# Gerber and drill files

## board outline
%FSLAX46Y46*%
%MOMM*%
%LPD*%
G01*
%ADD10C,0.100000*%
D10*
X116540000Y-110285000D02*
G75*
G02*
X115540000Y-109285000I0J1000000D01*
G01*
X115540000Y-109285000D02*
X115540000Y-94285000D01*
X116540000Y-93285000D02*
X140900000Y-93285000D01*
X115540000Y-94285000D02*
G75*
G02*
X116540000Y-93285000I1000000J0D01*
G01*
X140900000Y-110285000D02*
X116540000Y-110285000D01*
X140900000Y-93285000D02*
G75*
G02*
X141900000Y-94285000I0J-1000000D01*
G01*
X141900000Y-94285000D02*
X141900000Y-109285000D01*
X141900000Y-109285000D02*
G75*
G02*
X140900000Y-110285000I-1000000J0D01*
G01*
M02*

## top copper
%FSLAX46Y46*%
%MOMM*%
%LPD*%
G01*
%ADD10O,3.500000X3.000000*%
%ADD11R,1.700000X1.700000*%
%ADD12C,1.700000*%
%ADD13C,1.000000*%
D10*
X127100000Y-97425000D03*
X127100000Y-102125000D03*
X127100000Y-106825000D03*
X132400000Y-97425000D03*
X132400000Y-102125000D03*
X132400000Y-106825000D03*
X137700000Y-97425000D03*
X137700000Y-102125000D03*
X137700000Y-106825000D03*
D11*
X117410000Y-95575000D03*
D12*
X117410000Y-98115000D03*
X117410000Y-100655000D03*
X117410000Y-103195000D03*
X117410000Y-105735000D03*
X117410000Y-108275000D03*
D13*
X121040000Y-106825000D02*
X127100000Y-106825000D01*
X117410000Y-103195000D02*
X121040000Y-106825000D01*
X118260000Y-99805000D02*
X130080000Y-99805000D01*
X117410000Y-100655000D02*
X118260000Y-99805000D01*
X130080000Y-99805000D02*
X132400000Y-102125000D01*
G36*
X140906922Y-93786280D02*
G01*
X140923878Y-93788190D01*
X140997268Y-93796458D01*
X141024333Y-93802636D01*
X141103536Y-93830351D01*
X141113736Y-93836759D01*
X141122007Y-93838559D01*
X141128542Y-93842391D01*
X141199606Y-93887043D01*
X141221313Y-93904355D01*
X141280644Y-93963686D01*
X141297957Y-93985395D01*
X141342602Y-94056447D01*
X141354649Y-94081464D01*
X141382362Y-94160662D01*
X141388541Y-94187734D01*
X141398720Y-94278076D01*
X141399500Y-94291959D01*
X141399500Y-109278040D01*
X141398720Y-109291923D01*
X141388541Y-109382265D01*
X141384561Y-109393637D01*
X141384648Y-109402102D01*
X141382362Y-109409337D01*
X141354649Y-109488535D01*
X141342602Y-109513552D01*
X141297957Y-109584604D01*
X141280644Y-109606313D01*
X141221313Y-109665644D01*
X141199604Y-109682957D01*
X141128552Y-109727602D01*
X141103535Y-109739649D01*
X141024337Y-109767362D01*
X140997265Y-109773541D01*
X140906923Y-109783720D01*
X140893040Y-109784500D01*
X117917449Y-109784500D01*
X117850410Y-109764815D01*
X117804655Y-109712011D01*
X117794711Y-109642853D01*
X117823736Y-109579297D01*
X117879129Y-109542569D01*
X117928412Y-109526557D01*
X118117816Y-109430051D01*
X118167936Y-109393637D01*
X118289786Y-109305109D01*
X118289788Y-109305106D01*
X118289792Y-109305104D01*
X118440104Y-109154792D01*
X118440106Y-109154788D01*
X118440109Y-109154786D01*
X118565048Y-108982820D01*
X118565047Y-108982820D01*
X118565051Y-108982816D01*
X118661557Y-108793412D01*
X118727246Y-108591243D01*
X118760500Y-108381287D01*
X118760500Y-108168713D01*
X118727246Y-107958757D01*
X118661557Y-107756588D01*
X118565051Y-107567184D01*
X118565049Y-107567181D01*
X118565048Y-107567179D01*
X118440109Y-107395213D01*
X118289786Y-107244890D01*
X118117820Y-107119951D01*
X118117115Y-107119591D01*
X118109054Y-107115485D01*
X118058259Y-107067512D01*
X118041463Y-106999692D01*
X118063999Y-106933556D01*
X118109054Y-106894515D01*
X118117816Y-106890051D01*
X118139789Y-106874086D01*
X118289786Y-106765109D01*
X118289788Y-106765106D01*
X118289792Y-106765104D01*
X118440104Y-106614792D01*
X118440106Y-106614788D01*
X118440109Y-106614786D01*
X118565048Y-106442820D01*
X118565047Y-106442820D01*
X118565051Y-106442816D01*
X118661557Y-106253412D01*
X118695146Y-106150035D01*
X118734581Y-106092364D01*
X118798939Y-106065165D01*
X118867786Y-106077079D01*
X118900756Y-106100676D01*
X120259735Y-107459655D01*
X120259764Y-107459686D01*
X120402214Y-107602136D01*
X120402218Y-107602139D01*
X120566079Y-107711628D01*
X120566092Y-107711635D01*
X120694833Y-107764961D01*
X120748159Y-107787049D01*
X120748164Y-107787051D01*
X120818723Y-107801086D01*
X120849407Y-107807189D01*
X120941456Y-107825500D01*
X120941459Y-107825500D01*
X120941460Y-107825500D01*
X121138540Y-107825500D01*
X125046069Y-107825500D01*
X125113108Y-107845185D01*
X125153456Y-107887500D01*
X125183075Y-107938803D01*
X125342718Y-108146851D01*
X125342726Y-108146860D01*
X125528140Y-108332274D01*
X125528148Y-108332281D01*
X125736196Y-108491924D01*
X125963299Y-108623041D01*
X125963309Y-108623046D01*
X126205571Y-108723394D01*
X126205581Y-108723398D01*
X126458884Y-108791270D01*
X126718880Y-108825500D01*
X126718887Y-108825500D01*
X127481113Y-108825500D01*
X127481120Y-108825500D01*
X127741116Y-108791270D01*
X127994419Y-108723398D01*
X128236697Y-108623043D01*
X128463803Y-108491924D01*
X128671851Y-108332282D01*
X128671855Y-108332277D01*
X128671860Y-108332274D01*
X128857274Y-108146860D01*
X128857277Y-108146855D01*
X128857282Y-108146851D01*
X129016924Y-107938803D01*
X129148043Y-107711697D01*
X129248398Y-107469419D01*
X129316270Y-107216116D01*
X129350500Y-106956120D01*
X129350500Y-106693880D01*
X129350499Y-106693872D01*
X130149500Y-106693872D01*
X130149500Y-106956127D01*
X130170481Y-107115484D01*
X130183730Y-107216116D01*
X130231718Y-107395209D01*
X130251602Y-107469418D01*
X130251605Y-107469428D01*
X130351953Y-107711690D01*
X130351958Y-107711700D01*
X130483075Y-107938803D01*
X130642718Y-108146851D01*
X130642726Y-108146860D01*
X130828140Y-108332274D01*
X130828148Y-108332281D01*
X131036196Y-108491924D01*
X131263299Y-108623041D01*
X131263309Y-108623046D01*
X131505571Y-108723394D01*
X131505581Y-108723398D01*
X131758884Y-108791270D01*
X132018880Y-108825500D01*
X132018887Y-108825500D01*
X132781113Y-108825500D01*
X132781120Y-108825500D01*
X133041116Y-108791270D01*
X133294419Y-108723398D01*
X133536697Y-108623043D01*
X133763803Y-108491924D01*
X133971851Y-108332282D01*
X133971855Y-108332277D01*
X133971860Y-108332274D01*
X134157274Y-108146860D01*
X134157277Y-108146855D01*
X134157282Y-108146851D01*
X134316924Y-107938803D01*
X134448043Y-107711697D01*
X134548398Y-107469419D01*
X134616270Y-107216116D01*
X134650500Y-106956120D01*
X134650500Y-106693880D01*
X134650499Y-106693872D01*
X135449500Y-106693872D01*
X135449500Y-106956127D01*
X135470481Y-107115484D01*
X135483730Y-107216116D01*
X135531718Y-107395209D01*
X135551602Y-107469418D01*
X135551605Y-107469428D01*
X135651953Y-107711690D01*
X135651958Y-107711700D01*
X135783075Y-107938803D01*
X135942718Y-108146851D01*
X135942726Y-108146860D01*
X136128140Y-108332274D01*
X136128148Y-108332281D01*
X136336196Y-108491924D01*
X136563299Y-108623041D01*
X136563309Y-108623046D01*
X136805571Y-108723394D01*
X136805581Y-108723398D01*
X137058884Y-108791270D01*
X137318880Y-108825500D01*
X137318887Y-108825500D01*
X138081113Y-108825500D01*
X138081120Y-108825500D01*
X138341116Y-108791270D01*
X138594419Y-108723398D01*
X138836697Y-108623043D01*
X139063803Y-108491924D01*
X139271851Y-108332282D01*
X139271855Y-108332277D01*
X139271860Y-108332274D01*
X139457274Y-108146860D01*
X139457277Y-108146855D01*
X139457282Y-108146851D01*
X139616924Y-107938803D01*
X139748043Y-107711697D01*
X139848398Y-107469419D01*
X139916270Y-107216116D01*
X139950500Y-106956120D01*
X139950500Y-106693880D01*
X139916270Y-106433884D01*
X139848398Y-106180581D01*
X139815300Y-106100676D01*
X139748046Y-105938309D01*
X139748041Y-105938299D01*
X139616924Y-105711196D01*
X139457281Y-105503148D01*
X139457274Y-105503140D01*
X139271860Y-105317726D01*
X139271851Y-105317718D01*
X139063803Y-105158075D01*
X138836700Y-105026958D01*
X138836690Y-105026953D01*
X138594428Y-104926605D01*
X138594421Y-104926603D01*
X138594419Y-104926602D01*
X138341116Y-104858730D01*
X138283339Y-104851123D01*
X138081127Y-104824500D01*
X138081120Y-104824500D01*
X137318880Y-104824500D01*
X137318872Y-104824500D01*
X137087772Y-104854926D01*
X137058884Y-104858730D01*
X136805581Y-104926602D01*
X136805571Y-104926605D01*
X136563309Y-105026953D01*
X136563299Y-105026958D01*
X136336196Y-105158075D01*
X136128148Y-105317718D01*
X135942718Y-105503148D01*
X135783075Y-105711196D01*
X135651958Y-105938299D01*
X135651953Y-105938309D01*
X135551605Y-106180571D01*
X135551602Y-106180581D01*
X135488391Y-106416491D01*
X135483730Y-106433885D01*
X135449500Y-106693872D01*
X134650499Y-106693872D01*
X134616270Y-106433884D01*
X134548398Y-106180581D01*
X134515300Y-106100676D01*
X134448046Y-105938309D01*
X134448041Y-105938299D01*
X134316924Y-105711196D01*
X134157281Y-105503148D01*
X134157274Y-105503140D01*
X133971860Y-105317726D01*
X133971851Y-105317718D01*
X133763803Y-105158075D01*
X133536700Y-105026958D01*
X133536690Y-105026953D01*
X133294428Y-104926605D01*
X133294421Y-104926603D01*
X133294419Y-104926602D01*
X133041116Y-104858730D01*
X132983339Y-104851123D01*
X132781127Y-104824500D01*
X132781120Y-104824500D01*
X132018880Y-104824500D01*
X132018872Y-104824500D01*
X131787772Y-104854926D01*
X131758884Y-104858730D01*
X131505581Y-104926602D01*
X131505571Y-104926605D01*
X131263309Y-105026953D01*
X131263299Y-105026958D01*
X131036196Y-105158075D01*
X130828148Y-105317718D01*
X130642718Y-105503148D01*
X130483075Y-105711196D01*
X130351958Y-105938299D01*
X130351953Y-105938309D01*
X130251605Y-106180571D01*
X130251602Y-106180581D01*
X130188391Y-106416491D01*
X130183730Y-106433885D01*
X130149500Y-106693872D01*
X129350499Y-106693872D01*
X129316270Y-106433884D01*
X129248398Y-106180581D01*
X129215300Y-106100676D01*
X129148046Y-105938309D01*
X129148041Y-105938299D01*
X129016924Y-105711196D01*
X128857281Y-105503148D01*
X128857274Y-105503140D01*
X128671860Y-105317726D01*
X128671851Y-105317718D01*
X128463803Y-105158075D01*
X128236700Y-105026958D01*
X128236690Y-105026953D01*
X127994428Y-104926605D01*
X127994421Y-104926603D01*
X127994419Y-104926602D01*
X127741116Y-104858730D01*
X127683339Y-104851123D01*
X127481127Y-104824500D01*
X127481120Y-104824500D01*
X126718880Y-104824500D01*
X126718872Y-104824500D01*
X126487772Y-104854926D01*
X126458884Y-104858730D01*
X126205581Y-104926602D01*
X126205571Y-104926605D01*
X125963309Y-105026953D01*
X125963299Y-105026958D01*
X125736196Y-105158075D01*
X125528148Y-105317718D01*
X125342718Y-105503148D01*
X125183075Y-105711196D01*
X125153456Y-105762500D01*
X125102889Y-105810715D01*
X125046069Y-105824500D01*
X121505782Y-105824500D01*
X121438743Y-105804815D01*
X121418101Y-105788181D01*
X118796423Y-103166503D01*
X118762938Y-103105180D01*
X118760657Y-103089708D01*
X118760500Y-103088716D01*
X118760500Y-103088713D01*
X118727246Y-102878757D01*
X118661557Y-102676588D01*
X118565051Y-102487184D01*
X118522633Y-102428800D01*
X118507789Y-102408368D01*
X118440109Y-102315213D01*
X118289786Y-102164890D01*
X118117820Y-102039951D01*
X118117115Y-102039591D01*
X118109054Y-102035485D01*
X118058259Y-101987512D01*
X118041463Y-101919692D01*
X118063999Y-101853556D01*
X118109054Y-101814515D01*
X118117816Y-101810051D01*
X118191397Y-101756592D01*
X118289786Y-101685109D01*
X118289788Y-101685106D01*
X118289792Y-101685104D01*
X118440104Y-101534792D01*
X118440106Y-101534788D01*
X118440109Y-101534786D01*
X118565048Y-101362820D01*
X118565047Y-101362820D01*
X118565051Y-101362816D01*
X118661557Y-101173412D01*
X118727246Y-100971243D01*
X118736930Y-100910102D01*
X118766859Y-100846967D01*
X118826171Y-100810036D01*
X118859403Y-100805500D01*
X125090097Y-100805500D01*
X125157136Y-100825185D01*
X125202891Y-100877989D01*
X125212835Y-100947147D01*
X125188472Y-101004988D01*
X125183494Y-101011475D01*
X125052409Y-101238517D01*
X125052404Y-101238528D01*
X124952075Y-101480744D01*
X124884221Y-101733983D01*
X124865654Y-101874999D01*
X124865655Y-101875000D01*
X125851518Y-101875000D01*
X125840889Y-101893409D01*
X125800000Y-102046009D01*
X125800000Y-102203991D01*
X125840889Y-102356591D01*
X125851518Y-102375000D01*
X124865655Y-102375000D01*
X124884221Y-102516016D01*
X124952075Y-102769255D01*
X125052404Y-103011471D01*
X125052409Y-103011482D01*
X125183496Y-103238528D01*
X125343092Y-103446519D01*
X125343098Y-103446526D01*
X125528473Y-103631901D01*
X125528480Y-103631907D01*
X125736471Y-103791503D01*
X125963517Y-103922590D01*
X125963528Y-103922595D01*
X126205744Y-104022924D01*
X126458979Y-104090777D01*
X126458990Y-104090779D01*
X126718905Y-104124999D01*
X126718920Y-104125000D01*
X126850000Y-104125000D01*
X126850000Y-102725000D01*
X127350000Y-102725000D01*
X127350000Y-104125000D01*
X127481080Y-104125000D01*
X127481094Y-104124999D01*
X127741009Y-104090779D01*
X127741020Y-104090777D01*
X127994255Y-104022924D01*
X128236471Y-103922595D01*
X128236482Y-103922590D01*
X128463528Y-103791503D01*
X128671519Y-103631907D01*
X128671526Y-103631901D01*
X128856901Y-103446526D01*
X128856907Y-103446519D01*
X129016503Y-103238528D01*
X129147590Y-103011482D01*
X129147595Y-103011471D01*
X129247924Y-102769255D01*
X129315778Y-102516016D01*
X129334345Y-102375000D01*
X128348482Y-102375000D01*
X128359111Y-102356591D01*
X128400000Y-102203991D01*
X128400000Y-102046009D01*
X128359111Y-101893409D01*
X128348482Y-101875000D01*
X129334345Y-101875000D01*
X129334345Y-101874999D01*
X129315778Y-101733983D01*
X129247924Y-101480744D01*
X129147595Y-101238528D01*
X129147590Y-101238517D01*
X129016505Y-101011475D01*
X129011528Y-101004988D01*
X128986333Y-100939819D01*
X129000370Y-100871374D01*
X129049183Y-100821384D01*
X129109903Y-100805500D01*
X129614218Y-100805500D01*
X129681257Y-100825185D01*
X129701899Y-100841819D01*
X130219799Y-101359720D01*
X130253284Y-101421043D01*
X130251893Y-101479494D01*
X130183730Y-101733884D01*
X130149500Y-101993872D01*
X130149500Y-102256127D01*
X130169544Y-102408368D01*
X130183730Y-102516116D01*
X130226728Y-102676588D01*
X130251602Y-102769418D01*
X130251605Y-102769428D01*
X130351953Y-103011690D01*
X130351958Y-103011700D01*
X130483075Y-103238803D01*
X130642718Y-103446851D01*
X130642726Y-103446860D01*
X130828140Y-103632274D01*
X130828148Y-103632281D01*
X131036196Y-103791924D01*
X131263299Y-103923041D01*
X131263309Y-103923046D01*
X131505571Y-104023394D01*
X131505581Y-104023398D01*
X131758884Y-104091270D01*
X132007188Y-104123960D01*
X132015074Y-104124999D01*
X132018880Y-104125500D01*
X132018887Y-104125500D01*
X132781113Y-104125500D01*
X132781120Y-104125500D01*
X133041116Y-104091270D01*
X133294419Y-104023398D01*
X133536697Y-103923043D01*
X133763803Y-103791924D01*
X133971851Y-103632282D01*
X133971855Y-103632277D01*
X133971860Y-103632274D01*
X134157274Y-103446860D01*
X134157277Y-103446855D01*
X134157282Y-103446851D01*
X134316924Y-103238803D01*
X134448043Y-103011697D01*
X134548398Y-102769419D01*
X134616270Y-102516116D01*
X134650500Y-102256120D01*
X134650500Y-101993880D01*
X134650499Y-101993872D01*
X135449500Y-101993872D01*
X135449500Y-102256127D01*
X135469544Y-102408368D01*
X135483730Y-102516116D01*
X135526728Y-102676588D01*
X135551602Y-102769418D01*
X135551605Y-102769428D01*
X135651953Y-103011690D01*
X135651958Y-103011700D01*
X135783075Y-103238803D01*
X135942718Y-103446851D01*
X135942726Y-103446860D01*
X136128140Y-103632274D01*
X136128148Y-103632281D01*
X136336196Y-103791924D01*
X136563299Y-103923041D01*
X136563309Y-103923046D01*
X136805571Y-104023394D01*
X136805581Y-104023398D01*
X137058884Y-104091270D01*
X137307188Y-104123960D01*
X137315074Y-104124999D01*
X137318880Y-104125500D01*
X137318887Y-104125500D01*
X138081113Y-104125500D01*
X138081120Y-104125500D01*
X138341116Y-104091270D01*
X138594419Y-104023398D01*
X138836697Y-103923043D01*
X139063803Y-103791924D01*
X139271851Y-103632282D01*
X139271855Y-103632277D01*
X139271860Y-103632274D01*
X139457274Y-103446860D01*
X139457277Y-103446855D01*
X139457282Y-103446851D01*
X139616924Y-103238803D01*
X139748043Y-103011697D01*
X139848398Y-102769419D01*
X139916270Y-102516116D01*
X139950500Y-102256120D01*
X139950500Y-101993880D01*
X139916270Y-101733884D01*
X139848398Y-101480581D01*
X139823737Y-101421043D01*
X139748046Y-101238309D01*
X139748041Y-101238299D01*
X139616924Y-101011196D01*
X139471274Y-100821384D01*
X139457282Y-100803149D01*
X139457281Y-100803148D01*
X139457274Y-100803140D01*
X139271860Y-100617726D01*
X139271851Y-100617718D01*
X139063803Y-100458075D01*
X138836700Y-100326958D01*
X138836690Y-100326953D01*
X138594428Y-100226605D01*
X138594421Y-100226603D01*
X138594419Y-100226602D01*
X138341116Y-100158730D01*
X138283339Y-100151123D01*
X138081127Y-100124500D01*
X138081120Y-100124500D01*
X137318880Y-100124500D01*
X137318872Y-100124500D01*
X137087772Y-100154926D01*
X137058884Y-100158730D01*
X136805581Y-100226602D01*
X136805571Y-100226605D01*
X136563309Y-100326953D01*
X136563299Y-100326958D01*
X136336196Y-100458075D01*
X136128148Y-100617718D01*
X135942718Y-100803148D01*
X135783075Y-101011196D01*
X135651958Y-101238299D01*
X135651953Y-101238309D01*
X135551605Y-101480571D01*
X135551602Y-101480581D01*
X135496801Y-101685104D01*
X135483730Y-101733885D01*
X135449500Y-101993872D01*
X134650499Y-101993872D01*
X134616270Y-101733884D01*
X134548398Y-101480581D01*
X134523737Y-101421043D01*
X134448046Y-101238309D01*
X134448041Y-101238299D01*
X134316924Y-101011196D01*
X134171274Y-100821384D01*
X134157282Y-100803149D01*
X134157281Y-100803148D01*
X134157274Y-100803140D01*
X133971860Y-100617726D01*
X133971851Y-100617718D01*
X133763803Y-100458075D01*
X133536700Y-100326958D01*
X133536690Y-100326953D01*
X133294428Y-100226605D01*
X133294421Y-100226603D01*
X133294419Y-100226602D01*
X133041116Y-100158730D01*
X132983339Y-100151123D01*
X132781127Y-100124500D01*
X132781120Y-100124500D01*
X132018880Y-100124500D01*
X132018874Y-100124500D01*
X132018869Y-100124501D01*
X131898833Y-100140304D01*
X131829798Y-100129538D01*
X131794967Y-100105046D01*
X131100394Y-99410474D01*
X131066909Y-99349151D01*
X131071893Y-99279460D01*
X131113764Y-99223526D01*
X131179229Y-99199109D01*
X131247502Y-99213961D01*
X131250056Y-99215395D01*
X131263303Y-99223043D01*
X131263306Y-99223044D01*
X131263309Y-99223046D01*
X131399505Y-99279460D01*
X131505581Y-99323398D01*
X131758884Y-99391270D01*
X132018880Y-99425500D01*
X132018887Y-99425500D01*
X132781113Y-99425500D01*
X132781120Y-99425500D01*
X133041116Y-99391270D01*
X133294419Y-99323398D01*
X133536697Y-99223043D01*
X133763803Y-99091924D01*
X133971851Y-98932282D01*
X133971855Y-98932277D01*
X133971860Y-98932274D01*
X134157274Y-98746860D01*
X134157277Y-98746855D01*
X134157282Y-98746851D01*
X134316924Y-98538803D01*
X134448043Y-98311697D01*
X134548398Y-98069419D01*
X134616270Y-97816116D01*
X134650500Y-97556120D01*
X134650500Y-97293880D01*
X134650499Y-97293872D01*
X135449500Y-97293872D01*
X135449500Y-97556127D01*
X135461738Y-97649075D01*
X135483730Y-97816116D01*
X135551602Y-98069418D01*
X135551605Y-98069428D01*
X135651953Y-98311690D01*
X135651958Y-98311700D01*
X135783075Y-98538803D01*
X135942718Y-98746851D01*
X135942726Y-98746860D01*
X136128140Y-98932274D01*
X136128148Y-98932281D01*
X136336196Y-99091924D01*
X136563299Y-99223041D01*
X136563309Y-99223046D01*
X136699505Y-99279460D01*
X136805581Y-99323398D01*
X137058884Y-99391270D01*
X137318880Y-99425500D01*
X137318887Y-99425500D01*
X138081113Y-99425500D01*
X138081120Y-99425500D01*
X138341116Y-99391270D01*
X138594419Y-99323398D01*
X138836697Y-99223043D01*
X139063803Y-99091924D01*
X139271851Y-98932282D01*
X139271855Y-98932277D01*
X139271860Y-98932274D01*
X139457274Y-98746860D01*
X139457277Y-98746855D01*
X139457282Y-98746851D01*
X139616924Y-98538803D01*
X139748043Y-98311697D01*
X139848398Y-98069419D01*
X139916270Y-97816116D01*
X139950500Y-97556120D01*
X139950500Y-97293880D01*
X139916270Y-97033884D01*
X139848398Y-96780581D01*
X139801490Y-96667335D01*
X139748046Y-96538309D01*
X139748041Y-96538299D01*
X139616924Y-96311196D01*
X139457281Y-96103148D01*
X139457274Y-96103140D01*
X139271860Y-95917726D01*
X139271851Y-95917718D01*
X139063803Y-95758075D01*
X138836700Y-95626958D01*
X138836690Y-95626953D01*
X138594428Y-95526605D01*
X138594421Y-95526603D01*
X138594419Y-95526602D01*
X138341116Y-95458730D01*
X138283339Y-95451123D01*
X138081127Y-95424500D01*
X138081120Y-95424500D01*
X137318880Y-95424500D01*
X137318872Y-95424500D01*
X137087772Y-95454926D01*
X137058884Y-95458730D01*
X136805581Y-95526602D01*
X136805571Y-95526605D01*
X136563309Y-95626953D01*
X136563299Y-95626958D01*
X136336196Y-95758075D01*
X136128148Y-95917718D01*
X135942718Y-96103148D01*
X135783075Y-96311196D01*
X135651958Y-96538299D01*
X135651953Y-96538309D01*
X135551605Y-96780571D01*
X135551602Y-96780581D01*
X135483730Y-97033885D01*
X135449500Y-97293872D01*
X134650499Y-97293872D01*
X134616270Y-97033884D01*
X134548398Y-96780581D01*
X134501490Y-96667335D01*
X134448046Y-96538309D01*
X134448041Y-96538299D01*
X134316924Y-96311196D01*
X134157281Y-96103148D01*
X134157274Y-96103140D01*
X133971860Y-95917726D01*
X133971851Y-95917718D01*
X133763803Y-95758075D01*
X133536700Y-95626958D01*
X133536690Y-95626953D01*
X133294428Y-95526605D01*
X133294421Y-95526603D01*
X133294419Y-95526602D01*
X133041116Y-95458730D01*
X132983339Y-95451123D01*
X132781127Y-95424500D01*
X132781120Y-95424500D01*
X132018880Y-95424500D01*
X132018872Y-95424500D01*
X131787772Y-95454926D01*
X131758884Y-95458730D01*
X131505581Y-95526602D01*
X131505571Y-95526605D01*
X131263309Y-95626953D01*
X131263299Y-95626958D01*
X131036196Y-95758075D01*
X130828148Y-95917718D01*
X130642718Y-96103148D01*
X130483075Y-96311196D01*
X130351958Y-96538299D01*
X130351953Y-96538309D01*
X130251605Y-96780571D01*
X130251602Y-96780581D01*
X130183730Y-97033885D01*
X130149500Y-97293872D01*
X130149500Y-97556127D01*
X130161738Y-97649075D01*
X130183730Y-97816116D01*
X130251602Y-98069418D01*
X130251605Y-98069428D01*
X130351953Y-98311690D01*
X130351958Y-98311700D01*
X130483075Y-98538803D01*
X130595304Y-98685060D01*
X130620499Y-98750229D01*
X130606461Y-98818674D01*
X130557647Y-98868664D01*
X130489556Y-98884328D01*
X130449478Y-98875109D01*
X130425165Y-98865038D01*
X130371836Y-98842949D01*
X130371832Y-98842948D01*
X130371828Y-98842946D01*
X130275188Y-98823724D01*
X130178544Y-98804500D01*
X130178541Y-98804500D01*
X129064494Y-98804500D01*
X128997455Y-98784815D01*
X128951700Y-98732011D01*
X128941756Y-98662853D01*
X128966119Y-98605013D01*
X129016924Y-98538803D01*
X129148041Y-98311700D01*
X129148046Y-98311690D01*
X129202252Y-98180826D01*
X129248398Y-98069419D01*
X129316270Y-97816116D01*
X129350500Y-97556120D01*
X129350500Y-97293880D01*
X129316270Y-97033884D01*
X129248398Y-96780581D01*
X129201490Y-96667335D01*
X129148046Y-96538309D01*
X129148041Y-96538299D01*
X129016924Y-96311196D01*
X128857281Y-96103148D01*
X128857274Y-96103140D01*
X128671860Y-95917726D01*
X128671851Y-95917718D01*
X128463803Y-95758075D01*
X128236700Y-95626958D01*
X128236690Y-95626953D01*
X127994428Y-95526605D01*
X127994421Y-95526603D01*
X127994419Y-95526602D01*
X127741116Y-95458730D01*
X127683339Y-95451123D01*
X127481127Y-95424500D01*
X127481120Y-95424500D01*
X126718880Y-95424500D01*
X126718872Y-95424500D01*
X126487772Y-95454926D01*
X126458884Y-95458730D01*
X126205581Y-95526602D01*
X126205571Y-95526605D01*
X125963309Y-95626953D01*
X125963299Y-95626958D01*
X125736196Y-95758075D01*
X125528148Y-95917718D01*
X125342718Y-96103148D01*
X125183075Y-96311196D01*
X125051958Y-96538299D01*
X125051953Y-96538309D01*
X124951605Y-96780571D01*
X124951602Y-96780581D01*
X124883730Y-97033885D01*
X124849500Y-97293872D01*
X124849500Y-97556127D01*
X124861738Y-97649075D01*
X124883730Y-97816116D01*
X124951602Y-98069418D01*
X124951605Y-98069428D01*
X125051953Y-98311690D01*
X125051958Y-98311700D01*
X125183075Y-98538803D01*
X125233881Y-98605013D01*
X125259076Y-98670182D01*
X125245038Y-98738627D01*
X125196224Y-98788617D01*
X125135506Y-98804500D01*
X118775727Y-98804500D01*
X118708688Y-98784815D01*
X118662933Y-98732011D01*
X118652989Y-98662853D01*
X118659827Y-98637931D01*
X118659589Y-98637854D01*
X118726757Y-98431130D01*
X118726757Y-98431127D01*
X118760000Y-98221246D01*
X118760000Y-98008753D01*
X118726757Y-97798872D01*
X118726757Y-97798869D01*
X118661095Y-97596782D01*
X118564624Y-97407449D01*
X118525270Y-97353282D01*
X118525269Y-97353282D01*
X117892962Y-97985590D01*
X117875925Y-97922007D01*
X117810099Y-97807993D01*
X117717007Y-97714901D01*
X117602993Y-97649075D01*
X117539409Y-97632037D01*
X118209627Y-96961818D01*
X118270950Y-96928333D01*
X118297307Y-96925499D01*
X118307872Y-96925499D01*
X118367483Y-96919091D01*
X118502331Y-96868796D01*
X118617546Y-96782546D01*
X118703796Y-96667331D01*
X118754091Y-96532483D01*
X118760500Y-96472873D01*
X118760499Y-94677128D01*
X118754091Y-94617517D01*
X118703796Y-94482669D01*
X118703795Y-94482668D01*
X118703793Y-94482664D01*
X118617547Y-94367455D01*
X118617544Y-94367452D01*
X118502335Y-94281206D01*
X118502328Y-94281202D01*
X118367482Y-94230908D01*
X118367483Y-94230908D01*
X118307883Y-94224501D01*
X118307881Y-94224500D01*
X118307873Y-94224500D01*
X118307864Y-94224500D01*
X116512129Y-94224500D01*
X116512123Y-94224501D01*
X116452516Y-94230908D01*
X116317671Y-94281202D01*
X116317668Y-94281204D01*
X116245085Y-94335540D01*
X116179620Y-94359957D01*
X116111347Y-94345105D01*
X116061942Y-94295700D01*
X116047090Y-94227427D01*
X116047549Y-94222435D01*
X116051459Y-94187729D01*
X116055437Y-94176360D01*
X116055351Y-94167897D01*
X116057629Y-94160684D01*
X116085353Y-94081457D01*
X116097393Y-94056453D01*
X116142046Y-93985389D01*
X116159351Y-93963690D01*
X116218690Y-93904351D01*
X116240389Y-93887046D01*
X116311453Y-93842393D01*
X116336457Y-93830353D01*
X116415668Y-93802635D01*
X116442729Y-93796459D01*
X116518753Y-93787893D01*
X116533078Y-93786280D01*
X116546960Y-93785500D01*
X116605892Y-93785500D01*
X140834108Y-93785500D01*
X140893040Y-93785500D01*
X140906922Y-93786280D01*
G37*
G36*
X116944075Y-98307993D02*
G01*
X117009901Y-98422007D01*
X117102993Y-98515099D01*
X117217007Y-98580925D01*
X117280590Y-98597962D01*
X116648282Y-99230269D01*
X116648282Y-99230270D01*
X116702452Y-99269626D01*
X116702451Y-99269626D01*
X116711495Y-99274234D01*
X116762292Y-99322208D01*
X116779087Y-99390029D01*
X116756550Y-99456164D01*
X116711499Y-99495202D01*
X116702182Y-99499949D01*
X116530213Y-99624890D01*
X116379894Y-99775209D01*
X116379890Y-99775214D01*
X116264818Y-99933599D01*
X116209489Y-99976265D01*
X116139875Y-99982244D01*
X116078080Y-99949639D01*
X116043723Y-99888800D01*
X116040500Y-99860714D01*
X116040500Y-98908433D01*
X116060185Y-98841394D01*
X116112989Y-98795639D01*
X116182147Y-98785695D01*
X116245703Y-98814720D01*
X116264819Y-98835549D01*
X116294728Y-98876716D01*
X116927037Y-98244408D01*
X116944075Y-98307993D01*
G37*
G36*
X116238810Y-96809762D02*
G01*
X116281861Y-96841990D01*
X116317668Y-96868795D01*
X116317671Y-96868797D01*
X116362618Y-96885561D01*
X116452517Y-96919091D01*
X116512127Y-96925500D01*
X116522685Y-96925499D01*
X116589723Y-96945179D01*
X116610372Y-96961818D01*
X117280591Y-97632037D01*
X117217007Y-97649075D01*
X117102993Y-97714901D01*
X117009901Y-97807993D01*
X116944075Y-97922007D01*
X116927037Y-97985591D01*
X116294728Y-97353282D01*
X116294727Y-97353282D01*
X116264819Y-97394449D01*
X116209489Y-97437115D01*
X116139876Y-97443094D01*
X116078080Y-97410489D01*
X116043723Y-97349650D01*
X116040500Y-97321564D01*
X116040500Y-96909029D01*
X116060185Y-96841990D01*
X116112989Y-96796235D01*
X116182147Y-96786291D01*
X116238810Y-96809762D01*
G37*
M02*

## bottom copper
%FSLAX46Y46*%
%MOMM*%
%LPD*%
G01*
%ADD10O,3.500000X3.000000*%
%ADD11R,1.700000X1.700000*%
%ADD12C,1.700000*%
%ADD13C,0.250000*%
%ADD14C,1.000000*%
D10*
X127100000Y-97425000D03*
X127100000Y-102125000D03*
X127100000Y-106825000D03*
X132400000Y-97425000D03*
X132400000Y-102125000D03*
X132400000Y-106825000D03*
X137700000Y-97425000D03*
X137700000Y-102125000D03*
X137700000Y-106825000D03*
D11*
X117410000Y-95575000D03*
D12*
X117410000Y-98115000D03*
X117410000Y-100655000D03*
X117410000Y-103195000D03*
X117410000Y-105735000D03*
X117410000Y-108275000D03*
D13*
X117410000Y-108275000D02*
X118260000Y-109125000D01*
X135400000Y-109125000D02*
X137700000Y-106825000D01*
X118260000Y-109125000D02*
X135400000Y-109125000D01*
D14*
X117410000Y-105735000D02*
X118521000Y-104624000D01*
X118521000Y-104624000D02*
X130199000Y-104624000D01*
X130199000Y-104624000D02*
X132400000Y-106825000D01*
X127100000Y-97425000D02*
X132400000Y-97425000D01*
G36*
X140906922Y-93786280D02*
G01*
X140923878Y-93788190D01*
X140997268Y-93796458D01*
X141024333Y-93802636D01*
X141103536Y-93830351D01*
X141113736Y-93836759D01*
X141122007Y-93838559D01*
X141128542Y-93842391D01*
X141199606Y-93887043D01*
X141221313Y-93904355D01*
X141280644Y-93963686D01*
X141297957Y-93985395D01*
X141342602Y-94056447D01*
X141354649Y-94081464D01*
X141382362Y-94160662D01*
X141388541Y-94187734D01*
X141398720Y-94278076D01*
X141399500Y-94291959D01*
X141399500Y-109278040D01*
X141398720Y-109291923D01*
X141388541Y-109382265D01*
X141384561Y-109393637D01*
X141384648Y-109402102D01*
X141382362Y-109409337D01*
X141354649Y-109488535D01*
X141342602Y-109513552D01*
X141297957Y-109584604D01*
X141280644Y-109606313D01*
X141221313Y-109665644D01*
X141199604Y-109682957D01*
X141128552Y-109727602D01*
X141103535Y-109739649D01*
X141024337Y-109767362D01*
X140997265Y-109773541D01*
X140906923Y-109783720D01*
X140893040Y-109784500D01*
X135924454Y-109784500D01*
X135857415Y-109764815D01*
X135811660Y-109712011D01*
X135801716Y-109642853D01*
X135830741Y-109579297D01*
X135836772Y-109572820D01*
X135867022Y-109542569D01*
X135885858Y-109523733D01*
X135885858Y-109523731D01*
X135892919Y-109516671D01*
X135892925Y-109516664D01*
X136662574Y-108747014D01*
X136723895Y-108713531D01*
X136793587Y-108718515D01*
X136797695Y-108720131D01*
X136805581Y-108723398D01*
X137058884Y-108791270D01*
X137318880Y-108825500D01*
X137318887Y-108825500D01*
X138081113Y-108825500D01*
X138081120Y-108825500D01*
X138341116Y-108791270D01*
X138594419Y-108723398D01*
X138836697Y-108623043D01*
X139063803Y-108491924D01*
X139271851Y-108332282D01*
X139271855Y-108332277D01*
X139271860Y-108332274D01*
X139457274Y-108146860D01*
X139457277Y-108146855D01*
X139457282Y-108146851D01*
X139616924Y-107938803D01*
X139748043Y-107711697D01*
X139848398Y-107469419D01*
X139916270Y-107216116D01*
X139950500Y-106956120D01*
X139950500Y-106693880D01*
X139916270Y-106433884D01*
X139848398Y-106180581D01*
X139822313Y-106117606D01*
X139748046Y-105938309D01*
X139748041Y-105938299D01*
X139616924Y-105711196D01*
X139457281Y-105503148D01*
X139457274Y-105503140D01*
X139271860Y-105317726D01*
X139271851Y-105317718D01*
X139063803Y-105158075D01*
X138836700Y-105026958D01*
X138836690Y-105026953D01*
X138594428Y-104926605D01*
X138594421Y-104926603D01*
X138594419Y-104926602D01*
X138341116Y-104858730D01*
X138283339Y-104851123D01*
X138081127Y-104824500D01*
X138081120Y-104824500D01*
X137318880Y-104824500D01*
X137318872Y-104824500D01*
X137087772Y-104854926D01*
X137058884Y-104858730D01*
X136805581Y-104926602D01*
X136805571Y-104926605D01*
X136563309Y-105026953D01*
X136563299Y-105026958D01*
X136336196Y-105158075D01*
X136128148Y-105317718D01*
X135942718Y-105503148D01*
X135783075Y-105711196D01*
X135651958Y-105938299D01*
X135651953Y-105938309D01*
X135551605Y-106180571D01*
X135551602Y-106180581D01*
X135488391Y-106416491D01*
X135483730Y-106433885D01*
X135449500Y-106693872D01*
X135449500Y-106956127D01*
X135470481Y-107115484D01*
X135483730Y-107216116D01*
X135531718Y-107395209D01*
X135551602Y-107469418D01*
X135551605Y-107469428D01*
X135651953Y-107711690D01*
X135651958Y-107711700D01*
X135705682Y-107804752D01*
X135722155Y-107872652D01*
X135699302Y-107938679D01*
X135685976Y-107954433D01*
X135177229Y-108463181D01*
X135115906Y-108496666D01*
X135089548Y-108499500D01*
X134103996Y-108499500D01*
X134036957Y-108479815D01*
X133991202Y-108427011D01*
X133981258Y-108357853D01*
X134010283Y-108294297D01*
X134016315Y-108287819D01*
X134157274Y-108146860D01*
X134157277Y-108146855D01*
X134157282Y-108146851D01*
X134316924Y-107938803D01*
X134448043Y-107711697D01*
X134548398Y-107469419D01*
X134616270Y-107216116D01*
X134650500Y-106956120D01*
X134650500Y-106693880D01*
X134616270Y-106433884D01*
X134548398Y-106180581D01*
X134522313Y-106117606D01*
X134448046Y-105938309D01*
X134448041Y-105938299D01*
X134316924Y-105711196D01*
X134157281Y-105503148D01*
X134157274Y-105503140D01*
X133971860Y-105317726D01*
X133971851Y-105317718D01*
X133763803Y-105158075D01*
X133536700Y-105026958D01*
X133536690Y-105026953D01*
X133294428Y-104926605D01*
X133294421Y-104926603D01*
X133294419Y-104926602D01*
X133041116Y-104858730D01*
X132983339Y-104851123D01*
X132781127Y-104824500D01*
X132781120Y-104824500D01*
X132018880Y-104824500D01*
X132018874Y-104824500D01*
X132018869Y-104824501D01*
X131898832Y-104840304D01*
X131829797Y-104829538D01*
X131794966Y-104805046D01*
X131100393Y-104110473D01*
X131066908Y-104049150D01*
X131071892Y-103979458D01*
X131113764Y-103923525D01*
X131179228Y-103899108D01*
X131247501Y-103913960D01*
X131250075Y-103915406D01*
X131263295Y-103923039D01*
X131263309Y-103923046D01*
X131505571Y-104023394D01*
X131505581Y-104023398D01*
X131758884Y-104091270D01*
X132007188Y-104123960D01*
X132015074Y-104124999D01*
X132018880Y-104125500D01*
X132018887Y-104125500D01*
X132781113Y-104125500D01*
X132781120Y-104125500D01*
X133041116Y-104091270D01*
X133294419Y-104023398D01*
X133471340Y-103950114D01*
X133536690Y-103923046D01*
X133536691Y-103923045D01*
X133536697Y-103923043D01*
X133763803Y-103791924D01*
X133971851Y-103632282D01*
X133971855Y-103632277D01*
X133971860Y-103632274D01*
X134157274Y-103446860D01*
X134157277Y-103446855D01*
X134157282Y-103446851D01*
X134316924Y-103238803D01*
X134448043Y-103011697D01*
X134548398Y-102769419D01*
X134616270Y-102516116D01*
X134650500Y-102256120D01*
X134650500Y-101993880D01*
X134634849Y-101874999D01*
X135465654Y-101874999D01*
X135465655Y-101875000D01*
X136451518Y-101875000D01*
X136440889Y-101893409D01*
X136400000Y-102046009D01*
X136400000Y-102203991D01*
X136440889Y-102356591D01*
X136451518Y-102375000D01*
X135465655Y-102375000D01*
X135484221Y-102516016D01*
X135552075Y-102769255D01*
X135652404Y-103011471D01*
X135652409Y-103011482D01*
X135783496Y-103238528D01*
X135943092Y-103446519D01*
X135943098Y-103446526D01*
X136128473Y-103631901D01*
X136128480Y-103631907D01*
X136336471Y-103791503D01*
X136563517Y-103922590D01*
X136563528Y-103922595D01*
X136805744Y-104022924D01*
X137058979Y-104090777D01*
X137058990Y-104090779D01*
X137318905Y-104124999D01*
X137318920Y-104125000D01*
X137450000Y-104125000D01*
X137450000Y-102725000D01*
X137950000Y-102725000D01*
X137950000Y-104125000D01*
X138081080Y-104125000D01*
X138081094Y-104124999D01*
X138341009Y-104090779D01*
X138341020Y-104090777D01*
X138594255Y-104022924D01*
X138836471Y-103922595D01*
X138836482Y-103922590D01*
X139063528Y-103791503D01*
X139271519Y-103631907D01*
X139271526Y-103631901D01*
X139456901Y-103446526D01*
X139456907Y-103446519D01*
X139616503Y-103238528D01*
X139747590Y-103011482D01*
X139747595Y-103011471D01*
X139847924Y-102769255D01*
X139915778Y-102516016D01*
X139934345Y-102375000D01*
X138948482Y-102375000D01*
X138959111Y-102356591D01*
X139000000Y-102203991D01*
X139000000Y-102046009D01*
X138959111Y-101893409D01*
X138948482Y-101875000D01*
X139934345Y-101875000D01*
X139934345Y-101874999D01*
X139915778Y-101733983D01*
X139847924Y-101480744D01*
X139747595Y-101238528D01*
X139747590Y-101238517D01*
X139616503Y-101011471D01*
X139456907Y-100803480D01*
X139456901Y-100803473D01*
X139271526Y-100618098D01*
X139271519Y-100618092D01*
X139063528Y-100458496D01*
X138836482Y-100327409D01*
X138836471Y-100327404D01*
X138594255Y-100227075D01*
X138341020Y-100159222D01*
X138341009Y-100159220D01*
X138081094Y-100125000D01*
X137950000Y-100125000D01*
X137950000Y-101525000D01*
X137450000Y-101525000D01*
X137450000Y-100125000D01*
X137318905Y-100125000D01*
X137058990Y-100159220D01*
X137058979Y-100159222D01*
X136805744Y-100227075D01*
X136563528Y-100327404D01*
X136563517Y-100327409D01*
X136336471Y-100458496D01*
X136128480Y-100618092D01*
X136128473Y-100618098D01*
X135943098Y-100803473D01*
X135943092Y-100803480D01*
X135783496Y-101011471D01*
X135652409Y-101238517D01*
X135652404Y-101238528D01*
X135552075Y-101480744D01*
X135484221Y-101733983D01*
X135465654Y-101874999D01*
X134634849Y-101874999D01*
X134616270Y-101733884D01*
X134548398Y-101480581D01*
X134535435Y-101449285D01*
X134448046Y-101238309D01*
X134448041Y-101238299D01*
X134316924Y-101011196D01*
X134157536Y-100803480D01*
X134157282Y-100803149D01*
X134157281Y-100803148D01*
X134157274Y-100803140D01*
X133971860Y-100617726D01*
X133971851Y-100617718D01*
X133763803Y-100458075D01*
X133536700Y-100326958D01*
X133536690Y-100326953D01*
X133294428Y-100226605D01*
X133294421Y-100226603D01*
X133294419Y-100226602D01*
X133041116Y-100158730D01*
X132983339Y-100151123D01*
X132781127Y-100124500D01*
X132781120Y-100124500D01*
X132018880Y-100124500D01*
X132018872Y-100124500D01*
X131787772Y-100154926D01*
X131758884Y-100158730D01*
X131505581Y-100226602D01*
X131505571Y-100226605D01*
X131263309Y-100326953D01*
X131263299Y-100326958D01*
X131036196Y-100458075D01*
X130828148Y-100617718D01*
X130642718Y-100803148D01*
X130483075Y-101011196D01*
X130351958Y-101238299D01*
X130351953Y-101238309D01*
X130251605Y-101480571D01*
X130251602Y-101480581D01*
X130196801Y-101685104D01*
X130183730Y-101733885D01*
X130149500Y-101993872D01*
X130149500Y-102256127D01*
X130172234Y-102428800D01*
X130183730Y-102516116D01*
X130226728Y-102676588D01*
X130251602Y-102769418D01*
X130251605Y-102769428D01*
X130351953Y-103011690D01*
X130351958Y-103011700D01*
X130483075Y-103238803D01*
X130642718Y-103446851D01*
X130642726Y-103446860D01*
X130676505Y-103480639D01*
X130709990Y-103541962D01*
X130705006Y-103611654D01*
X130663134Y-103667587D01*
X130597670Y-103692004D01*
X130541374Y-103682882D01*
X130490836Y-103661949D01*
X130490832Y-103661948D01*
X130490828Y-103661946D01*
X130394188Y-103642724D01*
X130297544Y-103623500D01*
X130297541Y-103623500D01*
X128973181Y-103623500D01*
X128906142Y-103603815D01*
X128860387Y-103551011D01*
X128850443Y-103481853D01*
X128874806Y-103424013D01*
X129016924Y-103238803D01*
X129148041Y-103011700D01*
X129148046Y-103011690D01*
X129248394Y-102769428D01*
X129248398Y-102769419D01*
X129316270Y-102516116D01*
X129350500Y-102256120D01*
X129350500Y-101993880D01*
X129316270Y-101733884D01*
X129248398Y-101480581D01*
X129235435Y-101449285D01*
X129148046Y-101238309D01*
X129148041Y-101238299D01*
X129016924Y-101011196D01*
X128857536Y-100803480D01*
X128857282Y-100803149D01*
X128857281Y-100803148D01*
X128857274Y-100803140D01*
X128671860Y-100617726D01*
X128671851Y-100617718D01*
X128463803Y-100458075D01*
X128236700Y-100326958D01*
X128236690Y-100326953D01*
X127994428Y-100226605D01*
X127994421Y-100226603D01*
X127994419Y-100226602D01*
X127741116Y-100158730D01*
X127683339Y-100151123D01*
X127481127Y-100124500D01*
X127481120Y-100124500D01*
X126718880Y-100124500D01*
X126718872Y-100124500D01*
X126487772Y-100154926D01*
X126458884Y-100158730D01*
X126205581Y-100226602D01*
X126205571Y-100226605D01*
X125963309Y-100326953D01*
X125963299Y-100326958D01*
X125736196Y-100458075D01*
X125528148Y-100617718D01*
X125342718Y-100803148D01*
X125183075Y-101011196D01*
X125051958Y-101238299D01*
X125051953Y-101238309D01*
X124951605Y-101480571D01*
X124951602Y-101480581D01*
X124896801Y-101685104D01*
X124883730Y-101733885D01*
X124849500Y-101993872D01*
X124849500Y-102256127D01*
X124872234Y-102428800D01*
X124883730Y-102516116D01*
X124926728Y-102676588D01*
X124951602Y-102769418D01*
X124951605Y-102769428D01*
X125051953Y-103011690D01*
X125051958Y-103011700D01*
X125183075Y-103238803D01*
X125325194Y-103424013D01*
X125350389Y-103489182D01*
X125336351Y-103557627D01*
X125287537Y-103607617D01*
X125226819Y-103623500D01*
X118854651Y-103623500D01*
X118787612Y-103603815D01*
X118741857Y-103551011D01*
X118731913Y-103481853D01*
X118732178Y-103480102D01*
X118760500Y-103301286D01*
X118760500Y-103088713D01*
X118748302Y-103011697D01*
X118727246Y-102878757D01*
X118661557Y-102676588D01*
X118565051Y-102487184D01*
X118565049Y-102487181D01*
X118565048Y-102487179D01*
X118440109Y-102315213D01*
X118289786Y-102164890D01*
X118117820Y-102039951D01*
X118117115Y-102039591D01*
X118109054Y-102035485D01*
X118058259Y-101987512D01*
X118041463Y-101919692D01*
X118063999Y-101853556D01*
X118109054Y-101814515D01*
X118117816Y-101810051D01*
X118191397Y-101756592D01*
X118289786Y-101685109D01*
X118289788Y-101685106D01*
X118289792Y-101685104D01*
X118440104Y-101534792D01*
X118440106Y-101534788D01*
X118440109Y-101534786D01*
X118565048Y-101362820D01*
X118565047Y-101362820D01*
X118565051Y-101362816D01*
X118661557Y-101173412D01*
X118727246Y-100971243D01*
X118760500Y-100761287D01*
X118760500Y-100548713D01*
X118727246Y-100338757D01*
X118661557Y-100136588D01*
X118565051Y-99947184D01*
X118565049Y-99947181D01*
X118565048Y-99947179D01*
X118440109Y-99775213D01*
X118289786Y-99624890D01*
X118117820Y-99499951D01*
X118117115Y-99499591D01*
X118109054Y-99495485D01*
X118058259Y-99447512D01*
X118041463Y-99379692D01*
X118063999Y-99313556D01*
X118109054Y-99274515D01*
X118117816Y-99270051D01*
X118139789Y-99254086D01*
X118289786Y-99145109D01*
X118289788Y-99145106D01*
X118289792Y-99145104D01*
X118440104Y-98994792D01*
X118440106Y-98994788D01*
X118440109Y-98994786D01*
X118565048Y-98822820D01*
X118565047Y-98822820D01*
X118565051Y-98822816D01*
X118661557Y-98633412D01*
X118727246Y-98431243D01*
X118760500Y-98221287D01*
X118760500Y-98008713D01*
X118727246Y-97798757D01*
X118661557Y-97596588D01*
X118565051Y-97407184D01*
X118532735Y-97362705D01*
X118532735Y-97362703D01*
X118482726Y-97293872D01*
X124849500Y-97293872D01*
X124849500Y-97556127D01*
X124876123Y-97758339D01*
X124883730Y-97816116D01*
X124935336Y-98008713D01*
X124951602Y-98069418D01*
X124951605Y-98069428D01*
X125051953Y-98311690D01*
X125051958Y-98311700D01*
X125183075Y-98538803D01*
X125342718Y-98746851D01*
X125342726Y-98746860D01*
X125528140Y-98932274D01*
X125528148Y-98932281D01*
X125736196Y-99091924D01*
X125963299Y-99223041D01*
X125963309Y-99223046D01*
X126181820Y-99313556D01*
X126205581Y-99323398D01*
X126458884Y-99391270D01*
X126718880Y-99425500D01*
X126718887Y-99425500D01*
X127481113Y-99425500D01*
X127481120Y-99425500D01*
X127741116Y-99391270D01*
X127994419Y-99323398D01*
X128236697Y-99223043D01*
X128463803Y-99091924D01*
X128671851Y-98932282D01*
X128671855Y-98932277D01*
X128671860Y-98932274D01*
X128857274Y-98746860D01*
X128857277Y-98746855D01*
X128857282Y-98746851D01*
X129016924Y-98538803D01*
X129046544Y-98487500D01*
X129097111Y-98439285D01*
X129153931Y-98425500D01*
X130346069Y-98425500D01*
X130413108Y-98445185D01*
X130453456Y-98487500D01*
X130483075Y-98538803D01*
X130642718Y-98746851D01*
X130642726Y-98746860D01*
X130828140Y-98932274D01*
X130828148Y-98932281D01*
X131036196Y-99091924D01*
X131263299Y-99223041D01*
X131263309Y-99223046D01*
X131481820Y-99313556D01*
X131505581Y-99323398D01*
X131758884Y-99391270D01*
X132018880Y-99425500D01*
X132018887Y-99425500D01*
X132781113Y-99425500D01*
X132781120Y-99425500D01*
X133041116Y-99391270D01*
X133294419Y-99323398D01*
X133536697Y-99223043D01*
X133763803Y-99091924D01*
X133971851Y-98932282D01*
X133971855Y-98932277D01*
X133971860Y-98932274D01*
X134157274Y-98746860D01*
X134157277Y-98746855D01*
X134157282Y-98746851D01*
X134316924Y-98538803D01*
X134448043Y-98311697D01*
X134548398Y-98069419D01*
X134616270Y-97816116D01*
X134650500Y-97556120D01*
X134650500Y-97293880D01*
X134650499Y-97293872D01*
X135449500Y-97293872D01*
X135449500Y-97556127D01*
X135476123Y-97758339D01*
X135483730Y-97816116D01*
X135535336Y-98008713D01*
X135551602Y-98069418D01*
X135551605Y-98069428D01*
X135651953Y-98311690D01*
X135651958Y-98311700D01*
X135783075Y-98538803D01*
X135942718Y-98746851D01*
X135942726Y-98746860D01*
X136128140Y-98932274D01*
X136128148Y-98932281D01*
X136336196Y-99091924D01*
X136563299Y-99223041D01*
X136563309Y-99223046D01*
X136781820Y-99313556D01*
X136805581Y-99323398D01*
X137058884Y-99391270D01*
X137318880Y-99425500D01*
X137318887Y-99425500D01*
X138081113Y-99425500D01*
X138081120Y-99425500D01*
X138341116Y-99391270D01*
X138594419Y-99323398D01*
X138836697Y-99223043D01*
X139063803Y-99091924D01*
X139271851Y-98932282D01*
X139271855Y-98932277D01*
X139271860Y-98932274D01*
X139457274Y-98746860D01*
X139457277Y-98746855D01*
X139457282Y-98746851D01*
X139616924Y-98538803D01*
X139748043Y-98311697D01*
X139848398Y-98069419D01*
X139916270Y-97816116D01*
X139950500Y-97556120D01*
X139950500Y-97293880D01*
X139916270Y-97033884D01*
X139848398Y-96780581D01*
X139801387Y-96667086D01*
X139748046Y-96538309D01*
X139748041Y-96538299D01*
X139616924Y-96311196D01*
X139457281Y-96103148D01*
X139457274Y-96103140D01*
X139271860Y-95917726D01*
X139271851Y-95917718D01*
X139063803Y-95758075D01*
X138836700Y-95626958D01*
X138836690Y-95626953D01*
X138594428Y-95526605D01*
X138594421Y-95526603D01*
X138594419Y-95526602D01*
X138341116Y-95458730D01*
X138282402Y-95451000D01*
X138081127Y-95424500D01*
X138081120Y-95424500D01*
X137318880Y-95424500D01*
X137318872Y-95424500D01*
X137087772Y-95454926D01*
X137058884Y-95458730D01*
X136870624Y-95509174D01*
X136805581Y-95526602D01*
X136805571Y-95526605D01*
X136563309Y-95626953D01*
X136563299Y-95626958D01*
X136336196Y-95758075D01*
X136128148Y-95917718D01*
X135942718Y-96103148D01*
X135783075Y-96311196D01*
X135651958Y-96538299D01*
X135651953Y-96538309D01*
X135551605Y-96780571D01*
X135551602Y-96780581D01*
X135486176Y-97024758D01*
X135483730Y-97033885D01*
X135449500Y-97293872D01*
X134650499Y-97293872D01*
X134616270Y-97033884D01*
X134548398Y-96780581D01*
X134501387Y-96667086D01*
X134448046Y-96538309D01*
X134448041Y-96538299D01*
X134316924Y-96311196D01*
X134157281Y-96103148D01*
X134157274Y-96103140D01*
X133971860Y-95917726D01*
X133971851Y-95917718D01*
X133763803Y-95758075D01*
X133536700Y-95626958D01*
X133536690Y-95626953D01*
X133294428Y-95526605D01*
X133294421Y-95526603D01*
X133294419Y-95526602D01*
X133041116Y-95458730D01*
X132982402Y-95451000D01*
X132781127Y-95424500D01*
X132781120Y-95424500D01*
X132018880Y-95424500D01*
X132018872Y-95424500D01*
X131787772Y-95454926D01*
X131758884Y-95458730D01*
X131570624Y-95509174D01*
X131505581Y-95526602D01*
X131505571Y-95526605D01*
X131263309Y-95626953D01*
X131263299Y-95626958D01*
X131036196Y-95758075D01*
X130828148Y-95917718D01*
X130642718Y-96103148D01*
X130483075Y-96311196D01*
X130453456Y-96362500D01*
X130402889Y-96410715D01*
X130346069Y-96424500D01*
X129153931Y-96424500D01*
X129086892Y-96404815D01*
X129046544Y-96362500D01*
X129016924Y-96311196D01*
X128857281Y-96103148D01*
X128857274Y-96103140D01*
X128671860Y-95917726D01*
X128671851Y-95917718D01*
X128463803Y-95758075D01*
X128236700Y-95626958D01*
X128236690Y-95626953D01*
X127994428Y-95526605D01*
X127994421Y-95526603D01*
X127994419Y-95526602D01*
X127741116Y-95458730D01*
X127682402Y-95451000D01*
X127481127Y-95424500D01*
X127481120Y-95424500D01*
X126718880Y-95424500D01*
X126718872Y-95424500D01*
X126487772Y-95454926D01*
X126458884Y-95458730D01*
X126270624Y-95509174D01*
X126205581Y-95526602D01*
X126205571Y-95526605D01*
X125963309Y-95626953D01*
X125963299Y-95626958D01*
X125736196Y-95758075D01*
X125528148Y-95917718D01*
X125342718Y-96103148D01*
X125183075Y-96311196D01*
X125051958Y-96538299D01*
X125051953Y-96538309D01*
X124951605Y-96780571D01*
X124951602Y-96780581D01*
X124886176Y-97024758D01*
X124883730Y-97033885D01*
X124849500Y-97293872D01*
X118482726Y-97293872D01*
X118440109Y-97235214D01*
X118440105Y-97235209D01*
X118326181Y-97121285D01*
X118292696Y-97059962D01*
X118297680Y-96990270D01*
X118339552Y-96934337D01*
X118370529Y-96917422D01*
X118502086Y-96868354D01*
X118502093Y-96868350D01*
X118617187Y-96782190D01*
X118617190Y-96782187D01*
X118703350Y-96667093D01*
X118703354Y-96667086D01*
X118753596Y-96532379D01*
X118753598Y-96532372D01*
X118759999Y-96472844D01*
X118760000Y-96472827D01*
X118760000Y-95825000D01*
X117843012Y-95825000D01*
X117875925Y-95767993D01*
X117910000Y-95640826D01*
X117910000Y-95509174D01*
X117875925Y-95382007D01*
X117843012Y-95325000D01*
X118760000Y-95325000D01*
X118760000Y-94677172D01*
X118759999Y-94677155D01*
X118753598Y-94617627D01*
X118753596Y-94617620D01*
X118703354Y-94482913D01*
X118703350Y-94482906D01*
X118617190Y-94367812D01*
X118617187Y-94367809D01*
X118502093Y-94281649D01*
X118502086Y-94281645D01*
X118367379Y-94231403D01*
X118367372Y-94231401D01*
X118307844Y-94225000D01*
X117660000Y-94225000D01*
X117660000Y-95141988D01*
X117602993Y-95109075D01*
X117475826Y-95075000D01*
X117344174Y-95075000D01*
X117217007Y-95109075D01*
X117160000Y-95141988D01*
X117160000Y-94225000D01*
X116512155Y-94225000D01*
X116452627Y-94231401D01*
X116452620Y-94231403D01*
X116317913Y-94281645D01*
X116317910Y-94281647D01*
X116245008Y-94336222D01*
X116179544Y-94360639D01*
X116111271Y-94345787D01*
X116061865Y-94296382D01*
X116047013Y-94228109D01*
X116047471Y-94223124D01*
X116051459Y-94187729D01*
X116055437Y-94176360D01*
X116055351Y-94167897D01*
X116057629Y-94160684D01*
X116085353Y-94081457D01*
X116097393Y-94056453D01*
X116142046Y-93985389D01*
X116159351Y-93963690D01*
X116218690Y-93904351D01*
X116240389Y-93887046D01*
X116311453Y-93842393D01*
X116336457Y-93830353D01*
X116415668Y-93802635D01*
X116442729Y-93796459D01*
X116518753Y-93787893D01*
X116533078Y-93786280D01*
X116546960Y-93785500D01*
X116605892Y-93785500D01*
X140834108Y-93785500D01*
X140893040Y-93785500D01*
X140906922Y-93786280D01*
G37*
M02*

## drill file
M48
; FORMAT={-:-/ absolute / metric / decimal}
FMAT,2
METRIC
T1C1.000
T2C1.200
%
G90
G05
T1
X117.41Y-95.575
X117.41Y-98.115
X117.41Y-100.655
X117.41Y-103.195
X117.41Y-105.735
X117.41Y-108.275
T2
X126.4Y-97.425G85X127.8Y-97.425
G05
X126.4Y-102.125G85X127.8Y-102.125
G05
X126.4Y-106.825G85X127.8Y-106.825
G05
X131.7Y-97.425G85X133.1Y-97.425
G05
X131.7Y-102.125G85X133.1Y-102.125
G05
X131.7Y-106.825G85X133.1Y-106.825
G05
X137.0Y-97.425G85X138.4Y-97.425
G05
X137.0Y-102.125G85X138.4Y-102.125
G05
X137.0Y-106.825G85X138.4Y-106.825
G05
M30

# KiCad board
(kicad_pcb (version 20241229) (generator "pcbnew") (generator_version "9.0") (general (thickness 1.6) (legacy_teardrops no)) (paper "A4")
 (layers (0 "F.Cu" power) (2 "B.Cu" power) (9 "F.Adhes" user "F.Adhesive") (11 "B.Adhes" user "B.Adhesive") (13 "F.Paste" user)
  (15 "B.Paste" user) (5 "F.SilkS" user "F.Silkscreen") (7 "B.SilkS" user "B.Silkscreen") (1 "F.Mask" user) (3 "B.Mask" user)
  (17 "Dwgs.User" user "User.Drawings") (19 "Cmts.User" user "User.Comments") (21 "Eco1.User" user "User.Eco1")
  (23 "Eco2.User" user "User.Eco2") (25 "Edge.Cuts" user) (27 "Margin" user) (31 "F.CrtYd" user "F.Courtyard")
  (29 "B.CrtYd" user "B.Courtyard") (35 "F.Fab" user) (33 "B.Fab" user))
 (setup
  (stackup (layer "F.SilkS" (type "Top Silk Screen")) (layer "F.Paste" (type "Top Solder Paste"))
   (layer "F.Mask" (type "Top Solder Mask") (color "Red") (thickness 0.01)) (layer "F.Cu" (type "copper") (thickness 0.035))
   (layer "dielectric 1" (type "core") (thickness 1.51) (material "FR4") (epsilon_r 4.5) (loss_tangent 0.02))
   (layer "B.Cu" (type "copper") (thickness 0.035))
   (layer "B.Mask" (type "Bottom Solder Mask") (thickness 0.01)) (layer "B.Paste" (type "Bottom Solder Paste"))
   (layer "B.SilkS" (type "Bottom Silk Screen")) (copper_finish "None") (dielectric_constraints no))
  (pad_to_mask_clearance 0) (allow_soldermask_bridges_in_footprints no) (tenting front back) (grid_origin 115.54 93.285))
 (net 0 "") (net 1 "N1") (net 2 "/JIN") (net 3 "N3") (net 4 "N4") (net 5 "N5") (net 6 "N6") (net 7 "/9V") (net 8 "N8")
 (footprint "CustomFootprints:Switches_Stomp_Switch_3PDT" (layer "F.Cu") (at 132.1 101.785)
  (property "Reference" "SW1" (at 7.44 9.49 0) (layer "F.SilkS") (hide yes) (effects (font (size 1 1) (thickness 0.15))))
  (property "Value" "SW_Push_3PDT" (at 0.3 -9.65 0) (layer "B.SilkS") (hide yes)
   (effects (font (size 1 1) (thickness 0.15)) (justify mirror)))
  (pad "1" thru_hole oval (at -5 -4.36) (size 3.5 3) (drill oval 2.6 1.2) (layers "*.Cu" "*.Mask" "F.SilkS") (remove_unused_layers no)
   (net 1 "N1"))
  (pad "2" thru_hole oval (at -5 0.34) (size 3.5 3) (drill oval 2.6 1.2) (layers "*.Cu" "*.Mask" "F.SilkS") (remove_unused_layers no)
   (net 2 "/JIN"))
  (pad "3" thru_hole oval (at -5 5.04) (size 3.5 3) (drill oval 2.6 1.2) (layers "*.Cu" "*.Mask" "F.SilkS") (remove_unused_layers no)
   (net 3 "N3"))
  (pad "4" thru_hole oval (at 0.3 -4.36) (size 3.5 3) (drill oval 2.6 1.2) (layers "*.Cu" "*.Mask" "F.SilkS") (remove_unused_layers no)
   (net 1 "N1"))
  (pad "5" thru_hole oval (at 0.3 0.34) (size 3.5 3) (drill oval 2.6 1.2) (layers "*.Cu" "*.Mask" "F.SilkS") (remove_unused_layers no)
   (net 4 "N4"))
  (pad "6" thru_hole oval (at 0.3 5.04) (size 3.5 3) (drill oval 2.6 1.2) (layers "*.Cu" "*.Mask" "F.SilkS") (remove_unused_layers no)
   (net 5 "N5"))
  (pad "7" thru_hole oval (at 5.6 -4.36) (size 3.5 3) (drill oval 2.6 1.2) (layers "*.Cu" "*.Mask" "F.SilkS") (remove_unused_layers no)
   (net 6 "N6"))
  (pad "8" thru_hole oval (at 5.6 0.34) (size 3.5 3) (drill oval 2.6 1.2) (layers "*.Cu" "*.Mask" "F.SilkS") (remove_unused_layers no)
   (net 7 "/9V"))
  (pad "9" thru_hole oval (at 5.6 5.04) (size 3.5 3) (drill oval 2.6 1.2) (layers "*.Cu" "*.Mask" "F.SilkS") (remove_unused_layers no)
   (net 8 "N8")))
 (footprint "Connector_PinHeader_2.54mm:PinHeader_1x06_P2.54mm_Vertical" (layer "F.Cu") (at 117.41 95.575)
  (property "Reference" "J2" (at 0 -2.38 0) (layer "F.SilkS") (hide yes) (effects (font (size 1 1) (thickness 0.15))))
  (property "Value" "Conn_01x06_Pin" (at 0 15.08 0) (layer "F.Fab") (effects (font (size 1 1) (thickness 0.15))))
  (pad "1" thru_hole rect (at 0 0) (size 1.7 1.7) (drill 1) (layers "*.Cu" "*.Mask") (remove_unused_layers no) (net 7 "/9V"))
  (pad "2" thru_hole circle (at 0 2.54) (size 1.7 1.7) (drill 1) (layers "*.Cu" "*.Mask") (remove_unused_layers no) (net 2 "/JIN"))
  (pad "3" thru_hole circle (at 0 5.08) (size 1.7 1.7) (drill 1) (layers "*.Cu" "*.Mask") (remove_unused_layers no) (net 4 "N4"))
  (pad "4" thru_hole circle (at 0 7.62) (size 1.7 1.7) (drill 1) (layers "*.Cu" "*.Mask") (remove_unused_layers no) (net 3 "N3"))
  (pad "5" thru_hole circle (at 0 10.16) (size 1.7 1.7) (drill 1) (layers "*.Cu" "*.Mask") (remove_unused_layers no) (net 5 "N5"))
  (pad "6" thru_hole circle (at 0 12.7) (size 1.7 1.7) (drill 1) (layers "*.Cu" "*.Mask") (remove_unused_layers no) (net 8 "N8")))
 (gr_arc (start 116.54 110.285) (mid 115.832893 109.992107) (end 115.54 109.285) (stroke (width 0.1) (type default)) (layer "Edge.Cuts"))
 (gr_line (start 115.54 109.285) (end 115.54 94.285) (stroke (width 0.1) (type default)) (layer "Edge.Cuts"))
 (gr_line (start 116.54 93.285) (end 140.9 93.285) (stroke (width 0.1) (type default)) (layer "Edge.Cuts"))
 (gr_arc (start 115.54 94.285) (mid 115.832893 93.577893) (end 116.54 93.285) (stroke (width 0.1) (type default)) (layer "Edge.Cuts"))
 (gr_line (start 140.9 110.285) (end 116.54 110.285) (stroke (width 0.1) (type default)) (layer "Edge.Cuts"))
 (gr_arc (start 140.9 93.285) (mid 141.607107 93.577893) (end 141.9 94.285) (stroke (width 0.1) (type default)) (layer "Edge.Cuts"))
 (gr_line (start 141.9 94.285) (end 141.9 109.285) (stroke (width 0.1) (type default)) (layer "Edge.Cuts"))
 (gr_arc (start 141.9 109.285) (mid 141.607107 109.992107) (end 140.9 110.285) (stroke (width 0.1) (type default)) (layer "Edge.Cuts"))
 (segment (start 121.04 106.825) (end 127.1 106.825) (width 1) (layer "F.Cu") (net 3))
 (segment (start 117.41 103.195) (end 121.04 106.825) (width 1) (layer "F.Cu") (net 3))
 (segment (start 117.41 108.275) (end 118.26 109.125) (width 0.25) (layer "B.Cu") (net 8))
 (segment (start 135.4 109.125) (end 137.7 106.825) (width 0.25) (layer "B.Cu") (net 8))
 (segment (start 118.26 109.125) (end 135.4 109.125) (width 0.25) (layer "B.Cu") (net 8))
 (segment (start 118.26 99.805) (end 130.08 99.805) (width 1) (layer "F.Cu") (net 4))
 (segment (start 117.41 100.655) (end 118.26 99.805) (width 1) (layer "F.Cu") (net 4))
 (segment (start 130.08 99.805) (end 132.4 102.125) (width 1) (layer "F.Cu") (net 4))
 (segment (start 117.41 105.735) (end 118.521 104.624) (width 1) (layer "B.Cu") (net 5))
 (segment (start 118.521 104.624) (end 130.199 104.624) (width 1) (layer "B.Cu") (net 5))
 (segment (start 130.199 104.624) (end 132.4 106.825) (width 1) (layer "B.Cu") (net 5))
 (segment (start 127.1 97.425) (end 132.4 97.425) (width 1) (layer "B.Cu") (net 1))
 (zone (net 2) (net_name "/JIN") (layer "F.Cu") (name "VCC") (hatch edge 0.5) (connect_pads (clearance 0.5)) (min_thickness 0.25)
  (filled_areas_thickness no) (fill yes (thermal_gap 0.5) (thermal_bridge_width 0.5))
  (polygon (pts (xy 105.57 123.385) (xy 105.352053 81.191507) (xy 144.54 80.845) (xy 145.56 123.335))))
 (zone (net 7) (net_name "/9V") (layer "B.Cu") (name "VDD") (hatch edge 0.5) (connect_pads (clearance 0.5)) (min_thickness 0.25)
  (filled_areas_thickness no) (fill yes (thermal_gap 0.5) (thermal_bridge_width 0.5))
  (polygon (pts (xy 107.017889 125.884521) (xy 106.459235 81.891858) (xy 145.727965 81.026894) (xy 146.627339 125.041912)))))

